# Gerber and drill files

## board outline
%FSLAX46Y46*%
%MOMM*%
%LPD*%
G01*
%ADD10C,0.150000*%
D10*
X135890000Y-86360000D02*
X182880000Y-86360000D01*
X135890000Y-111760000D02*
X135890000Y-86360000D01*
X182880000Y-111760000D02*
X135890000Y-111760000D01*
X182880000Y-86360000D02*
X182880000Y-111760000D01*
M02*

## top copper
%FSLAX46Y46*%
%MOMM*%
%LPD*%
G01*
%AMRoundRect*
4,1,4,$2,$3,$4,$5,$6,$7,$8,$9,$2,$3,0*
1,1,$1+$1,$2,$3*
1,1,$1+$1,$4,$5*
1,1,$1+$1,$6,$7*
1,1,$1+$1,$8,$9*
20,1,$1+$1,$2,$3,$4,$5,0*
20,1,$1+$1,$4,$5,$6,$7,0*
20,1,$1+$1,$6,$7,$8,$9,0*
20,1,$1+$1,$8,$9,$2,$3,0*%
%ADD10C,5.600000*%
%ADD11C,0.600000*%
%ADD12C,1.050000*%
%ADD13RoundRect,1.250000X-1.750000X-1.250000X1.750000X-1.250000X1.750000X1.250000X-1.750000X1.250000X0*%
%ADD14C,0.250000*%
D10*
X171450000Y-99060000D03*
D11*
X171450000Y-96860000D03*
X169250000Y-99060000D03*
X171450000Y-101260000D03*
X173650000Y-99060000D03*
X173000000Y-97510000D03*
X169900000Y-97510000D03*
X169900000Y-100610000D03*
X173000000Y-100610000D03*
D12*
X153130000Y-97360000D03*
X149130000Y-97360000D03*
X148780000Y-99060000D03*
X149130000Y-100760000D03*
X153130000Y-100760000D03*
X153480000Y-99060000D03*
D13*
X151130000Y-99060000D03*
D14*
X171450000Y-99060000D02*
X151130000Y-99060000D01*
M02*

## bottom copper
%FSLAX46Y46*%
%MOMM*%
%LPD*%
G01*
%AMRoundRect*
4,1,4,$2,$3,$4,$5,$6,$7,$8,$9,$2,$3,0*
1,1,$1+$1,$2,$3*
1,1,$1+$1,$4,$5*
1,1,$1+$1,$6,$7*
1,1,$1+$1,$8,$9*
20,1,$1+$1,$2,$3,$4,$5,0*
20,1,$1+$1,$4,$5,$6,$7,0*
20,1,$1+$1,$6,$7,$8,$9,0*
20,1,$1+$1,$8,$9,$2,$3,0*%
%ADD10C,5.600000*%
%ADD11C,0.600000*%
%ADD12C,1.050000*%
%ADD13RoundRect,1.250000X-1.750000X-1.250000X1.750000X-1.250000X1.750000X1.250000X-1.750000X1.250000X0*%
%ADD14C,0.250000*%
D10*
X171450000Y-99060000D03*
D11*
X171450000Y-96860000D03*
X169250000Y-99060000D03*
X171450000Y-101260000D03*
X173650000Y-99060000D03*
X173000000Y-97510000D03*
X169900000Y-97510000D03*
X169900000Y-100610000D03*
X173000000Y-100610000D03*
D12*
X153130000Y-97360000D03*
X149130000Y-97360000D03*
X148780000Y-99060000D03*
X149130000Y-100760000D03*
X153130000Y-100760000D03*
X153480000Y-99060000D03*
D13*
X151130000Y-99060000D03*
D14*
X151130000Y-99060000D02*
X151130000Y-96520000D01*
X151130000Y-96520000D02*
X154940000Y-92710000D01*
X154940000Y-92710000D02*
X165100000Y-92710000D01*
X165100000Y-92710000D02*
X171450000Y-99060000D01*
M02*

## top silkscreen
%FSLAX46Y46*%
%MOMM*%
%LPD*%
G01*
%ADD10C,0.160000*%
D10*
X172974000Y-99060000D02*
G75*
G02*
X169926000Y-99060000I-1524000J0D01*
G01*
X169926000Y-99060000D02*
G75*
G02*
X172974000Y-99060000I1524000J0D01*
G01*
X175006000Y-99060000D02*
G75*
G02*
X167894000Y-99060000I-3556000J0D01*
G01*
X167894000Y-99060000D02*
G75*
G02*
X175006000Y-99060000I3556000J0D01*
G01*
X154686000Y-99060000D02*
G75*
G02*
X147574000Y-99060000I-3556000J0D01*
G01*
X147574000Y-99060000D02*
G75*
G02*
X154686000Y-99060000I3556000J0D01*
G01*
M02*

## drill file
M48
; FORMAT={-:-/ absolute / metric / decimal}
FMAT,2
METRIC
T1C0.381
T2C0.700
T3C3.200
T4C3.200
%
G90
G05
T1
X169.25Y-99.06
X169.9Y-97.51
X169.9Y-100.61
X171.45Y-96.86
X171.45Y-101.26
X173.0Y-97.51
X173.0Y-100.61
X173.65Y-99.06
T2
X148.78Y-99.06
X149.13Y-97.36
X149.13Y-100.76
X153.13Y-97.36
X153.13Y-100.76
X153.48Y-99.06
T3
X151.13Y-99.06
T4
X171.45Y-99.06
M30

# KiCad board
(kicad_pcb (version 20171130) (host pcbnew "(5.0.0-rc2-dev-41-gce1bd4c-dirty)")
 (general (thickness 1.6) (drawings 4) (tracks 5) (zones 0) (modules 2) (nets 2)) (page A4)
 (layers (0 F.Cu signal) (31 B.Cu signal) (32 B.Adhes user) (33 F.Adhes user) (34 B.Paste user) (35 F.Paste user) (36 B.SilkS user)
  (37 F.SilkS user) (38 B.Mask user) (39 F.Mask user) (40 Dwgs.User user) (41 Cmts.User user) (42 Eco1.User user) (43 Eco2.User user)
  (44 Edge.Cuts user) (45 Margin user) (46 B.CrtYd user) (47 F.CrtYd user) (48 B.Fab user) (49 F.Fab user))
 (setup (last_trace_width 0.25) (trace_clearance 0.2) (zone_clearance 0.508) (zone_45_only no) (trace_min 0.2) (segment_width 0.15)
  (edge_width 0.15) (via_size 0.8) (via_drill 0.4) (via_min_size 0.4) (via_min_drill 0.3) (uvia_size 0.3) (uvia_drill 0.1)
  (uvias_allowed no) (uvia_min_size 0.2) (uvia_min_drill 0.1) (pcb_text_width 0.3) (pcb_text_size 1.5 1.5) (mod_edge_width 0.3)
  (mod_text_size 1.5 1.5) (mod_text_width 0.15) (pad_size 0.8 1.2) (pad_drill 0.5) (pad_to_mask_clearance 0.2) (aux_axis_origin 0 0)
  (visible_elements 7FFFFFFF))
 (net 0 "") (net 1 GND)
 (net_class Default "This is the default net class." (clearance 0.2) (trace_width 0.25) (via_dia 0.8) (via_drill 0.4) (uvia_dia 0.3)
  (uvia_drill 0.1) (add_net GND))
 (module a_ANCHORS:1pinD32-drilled (layer F.Cu) (at 171.45 99.06)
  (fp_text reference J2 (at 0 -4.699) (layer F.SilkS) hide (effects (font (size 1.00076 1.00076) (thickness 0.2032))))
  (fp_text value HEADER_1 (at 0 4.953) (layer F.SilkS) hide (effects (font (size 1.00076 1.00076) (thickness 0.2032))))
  (fp_circle (center 0 0) (end 0 1.524) (layer F.SilkS) (width 0.16))
  (fp_circle (center 0 0) (end 0 3.556) (layer F.SilkS) (width 0.16))
  (pad 1 thru_hole circle (at 0 0) (size 5.6 5.6) (drill 3.2004) (layers *.Cu *.Mask) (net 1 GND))
  (pad 1 thru_hole circle (at 0 -2.2) (size 0.6 0.6) (drill 0.381) (layers *.Cu *.Mask) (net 1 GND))
  (pad 1 thru_hole circle (at -2.2 0) (size 0.6 0.6) (drill 0.381) (layers *.Cu *.Mask) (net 1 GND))
  (pad 1 thru_hole circle (at 0 2.2) (size 0.6 0.6) (drill 0.381) (layers *.Cu *.Mask) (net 1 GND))
  (pad 1 thru_hole circle (at 2.2 0) (size 0.6 0.6) (drill 0.381) (layers *.Cu *.Mask) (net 1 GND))
  (pad 1 thru_hole circle (at 1.55 -1.55) (size 0.6 0.6) (drill 0.381) (layers *.Cu *.Mask) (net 1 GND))
  (pad 1 thru_hole circle (at -1.55 -1.55) (size 0.6 0.6) (drill 0.381) (layers *.Cu *.Mask) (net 1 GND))
  (pad 1 thru_hole circle (at -1.55 1.55) (size 0.6 0.6) (drill 0.381) (layers *.Cu *.Mask) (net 1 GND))
  (pad 1 thru_hole circle (at 1.55 1.55) (size 0.6 0.6) (drill 0.381) (layers *.Cu *.Mask) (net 1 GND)))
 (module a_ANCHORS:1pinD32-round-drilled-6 (layer F.Cu) (at 151.13 99.06)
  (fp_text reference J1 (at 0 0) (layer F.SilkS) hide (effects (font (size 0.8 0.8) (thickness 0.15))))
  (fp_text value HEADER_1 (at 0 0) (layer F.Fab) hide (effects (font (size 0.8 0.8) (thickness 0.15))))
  (fp_circle (center 0 0) (end 0 3.556) (layer F.SilkS) (width 0.16))
  (pad 1 thru_hole circle (at 2 -1.7) (size 1.05 1.05) (drill 0.7) (layers *.Cu *.Mask) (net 1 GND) (zone_connect 2))
  (pad 1 thru_hole circle (at -2 -1.7) (size 1.05 1.05) (drill 0.7) (layers *.Cu *.Mask) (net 1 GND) (zone_connect 2))
  (pad 1 thru_hole circle (at -2.35 0) (size 1.05 1.05) (drill 0.7) (layers *.Cu *.Mask) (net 1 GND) (zone_connect 2))
  (pad 1 thru_hole circle (at -2 1.7) (size 1.05 1.05) (drill 0.7) (layers *.Cu *.Mask) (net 1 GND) (zone_connect 2))
  (pad 1 thru_hole circle (at 2 1.7) (size 1.05 1.05) (drill 0.7) (layers *.Cu *.Mask) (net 1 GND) (zone_connect 2))
  (pad 1 thru_hole circle (at 2.35 0) (size 1.05 1.05) (drill 0.7) (layers *.Cu *.Mask) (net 1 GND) (zone_connect 2))
  (pad 1 thru_hole roundrect (at 0 0) (size 6 5) (drill 3.2) (layers *.Cu *.Mask) (roundrect_rratio 0.25) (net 1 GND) (zone_connect 2)))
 (gr_line (start 135.89 86.36) (end 182.88 86.36) (angle 90) (layer Edge.Cuts) (width 0.15))
 (gr_line (start 135.89 111.76) (end 135.89 86.36) (angle 90) (layer Edge.Cuts) (width 0.15))
 (gr_line (start 182.88 111.76) (end 135.89 111.76) (angle 90) (layer Edge.Cuts) (width 0.15))
 (gr_line (start 182.88 86.36) (end 182.88 111.76) (angle 90) (layer Edge.Cuts) (width 0.15))
 (segment (start 151.13 99.06) (end 151.13 96.52) (width 0.25) (layer B.Cu) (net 1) (status 400000))
 (segment (start 151.13 96.52) (end 154.94 92.71) (width 0.25) (layer B.Cu) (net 1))
 (segment (start 154.94 92.71) (end 165.1 92.71) (width 0.25) (layer B.Cu) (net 1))
 (segment (start 165.1 92.71) (end 171.45 99.06) (width 0.25) (layer B.Cu) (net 1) (status 800000))
 (segment (start 171.45 99.06) (end 151.13 99.06) (width 0.25) (layer F.Cu) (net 1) (status C00000)))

